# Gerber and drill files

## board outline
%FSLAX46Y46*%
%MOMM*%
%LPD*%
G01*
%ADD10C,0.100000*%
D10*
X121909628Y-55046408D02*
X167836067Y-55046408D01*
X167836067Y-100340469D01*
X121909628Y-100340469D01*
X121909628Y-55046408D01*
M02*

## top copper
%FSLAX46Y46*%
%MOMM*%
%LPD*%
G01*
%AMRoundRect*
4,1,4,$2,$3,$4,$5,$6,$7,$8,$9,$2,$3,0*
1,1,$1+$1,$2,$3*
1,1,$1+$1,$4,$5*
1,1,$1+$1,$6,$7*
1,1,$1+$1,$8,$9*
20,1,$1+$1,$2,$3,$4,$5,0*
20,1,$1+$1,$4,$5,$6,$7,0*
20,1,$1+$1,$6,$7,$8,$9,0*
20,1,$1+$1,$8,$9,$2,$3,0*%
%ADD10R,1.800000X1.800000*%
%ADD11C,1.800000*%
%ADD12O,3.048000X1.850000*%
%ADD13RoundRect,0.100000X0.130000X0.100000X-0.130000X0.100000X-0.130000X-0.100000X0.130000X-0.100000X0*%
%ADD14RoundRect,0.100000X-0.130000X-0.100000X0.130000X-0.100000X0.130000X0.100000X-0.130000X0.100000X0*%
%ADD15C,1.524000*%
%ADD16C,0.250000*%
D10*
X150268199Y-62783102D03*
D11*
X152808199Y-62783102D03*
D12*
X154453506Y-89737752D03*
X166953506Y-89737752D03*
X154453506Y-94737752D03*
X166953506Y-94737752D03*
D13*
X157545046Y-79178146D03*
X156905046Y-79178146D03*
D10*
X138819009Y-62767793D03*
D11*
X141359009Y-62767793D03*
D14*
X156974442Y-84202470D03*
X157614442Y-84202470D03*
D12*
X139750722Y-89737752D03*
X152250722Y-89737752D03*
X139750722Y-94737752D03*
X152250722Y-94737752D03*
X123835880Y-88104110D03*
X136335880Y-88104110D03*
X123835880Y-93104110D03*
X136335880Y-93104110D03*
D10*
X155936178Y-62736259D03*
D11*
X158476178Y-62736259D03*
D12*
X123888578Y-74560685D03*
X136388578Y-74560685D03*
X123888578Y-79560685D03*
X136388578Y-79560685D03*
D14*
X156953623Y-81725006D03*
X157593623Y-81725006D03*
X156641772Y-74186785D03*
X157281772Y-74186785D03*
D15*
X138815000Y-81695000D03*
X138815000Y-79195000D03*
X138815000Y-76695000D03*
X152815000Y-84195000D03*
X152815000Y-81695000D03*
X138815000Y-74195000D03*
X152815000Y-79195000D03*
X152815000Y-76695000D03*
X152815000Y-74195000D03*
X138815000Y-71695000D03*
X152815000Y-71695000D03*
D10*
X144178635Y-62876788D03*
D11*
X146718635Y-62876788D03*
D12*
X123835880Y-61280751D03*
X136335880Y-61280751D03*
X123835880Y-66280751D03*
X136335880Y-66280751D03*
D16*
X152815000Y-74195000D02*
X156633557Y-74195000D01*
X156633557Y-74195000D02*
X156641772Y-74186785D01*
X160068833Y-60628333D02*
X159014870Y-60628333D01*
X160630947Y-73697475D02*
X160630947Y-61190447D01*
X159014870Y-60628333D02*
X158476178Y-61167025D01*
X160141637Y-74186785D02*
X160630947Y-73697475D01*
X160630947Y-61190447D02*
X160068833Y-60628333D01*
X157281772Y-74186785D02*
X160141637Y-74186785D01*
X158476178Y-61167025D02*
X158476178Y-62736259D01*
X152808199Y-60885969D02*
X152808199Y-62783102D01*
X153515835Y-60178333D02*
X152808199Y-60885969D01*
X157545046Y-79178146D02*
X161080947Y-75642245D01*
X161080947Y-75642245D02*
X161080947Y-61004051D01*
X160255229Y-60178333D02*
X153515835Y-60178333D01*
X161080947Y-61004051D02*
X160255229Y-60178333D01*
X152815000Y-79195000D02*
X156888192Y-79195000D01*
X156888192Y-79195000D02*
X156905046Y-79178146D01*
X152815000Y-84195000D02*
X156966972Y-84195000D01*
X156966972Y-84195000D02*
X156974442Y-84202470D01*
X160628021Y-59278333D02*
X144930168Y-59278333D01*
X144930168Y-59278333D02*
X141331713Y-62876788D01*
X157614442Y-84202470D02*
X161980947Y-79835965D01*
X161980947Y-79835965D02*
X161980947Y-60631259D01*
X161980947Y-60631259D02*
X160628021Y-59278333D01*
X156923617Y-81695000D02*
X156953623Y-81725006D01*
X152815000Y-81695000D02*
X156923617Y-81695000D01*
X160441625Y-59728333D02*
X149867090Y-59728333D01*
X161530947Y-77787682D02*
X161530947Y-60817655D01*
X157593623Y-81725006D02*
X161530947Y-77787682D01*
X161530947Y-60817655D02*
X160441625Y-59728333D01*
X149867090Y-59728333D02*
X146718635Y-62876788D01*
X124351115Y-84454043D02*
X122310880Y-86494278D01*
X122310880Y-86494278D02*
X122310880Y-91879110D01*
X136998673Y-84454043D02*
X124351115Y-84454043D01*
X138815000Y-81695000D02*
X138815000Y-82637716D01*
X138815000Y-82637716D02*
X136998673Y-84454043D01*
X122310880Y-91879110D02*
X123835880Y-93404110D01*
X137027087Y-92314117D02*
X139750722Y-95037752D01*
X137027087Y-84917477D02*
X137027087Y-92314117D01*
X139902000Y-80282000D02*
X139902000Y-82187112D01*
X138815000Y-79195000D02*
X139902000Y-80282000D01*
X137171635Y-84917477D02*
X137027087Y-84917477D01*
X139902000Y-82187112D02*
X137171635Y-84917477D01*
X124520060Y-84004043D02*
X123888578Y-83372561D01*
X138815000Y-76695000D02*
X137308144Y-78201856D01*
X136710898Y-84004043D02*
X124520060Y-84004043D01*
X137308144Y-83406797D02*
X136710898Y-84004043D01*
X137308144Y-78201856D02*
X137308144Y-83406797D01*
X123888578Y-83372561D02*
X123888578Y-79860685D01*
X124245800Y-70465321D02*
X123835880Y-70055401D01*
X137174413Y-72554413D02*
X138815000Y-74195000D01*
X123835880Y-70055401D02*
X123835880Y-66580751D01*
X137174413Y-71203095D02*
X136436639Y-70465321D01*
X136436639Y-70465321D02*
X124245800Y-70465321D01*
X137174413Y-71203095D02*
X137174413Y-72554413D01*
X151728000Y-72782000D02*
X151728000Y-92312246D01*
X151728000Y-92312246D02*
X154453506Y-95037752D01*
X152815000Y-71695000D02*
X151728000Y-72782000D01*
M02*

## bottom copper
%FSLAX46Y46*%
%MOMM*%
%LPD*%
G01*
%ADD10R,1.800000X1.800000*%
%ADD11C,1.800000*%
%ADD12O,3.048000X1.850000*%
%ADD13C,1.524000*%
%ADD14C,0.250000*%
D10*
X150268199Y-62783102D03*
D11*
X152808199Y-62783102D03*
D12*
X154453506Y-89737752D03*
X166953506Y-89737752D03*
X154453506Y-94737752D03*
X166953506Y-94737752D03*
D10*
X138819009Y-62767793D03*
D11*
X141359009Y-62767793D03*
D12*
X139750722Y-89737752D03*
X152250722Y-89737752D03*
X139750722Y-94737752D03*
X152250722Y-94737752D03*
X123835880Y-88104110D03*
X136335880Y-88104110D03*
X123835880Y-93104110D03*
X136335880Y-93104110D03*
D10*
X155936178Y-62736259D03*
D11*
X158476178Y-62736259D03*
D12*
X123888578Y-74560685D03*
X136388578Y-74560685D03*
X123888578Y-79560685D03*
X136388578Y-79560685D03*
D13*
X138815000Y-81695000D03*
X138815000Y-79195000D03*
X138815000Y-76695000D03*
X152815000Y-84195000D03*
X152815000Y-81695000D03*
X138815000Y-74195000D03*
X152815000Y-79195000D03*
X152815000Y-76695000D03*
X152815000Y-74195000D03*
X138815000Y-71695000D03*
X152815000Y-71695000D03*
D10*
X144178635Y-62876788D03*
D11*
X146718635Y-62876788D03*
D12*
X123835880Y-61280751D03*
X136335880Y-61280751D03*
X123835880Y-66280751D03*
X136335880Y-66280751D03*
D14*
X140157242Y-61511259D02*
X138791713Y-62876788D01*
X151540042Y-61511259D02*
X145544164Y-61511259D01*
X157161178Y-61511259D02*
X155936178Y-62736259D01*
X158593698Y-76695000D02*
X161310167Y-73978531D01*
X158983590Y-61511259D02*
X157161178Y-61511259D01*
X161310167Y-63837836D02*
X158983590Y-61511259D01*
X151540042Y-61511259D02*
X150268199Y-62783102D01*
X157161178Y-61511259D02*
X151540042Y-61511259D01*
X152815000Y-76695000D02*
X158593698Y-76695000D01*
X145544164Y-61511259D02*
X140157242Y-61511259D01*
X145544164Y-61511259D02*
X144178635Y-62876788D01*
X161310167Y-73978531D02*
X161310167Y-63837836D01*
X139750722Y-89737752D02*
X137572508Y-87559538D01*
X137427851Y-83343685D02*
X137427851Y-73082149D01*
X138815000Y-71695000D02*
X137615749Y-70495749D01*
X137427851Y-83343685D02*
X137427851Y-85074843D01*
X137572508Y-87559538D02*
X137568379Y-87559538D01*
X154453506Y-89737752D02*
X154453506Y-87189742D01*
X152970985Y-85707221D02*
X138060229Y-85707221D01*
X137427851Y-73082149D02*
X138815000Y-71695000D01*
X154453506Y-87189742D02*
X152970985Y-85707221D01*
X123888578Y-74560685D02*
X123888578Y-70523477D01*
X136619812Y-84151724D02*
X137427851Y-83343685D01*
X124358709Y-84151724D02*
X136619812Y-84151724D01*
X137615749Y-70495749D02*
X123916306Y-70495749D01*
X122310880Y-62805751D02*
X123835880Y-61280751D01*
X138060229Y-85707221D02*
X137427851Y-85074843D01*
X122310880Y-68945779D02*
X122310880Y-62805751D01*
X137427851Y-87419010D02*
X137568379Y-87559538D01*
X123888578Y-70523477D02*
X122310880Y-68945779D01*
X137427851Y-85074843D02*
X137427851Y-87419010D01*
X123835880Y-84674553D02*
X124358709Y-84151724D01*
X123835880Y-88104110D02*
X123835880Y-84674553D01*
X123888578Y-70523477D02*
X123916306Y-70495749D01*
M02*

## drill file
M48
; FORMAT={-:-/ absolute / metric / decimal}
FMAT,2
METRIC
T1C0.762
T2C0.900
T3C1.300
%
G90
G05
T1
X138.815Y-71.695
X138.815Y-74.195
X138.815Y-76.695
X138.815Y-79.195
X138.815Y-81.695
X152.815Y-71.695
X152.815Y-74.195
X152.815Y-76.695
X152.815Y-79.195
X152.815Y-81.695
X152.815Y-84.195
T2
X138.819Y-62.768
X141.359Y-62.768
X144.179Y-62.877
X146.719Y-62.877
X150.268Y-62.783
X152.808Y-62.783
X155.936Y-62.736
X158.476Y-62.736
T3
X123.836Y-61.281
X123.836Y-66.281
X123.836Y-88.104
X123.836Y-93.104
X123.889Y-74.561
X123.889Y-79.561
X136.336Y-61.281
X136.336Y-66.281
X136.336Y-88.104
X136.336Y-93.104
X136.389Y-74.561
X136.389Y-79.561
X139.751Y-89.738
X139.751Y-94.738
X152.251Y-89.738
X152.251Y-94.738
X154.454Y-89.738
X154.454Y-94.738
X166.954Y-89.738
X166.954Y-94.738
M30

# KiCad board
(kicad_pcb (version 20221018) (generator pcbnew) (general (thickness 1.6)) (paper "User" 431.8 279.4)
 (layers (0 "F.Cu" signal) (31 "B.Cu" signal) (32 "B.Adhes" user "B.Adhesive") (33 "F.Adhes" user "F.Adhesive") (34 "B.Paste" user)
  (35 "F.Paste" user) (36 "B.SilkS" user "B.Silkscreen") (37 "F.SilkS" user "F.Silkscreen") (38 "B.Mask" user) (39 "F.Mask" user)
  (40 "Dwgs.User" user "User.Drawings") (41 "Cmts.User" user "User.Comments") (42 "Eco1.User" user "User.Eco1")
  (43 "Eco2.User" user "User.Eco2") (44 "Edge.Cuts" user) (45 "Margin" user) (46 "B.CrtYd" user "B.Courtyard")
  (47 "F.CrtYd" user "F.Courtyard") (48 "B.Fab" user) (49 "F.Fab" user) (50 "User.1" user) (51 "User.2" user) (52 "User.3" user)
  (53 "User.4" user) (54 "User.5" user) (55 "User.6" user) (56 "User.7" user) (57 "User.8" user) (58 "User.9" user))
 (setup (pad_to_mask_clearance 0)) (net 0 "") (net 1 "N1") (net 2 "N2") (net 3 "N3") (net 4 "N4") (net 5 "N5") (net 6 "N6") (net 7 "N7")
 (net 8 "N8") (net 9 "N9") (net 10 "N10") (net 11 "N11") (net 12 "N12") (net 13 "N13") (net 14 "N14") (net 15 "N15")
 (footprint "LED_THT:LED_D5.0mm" (layer "F.Cu") (at 150.268199 62.783102)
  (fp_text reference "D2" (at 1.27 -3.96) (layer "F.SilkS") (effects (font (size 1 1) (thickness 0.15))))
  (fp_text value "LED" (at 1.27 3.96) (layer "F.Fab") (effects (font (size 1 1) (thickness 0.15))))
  (pad "1" thru_hole rect (at 0 0) (size 1.8 1.8) (drill 0.9) (layers "*.Cu" "*.Mask") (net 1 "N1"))
  (pad "2" thru_hole circle (at 2.54 0) (size 1.8 1.8) (drill 0.9) (layers "*.Cu" "*.Mask") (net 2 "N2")))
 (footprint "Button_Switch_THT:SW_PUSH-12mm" (layer "F.Cu") (at 154.453506 89.737752)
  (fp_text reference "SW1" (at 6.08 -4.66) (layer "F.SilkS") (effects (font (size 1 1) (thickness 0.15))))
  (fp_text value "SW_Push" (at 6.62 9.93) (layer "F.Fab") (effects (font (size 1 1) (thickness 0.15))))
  (pad "1" thru_hole oval (at 0 0) (size 3.048 1.85) (drill 1.3) (layers "*.Cu" "*.Mask") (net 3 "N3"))
  (pad "1" thru_hole oval (at 12.5 0) (size 3.048 1.85) (drill 1.3) (layers "*.Cu" "*.Mask") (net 3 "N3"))
  (pad "2" thru_hole oval (at 0 5) (size 3.048 1.85) (drill 1.3) (layers "*.Cu" "*.Mask") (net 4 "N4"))
  (pad "2" thru_hole oval (at 12.5 5) (size 3.048 1.85) (drill 1.3) (layers "*.Cu" "*.Mask") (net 4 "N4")))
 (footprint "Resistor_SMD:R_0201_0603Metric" (layer "F.Cu") (at 157.225046 79.178146 180)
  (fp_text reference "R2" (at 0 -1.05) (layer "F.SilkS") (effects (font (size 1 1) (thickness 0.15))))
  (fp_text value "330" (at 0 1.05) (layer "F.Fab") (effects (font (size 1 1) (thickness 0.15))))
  (pad "" smd roundrect (at -0.345 0 180) (size 0.318 0.36) (layers "F.Paste") (roundrect_rratio 0.25))
  (pad "" smd roundrect (at 0.345 0 180) (size 0.318 0.36) (layers "F.Paste") (roundrect_rratio 0.25))
  (pad "1" smd roundrect (at -0.32 0 180) (size 0.46 0.4) (layers "F.Cu" "F.Mask") (roundrect_rratio 0.25) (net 2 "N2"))
  (pad "2" smd roundrect (at 0.32 0 180) (size 0.46 0.4) (layers "F.Cu" "F.Mask") (roundrect_rratio 0.25) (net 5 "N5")))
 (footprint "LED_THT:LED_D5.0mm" (layer "F.Cu") (at 138.819009 62.767793)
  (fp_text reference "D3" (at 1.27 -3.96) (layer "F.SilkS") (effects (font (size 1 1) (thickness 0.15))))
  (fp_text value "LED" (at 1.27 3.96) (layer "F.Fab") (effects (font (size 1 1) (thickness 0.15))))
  (pad "1" thru_hole rect (at 0 0) (size 1.8 1.8) (drill 0.9) (layers "*.Cu" "*.Mask") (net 1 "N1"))
  (pad "2" thru_hole circle (at 2.54 0) (size 1.8 1.8) (drill 0.9) (layers "*.Cu" "*.Mask") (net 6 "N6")))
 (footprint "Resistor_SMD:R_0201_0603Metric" (layer "F.Cu") (at 157.294442 84.20247)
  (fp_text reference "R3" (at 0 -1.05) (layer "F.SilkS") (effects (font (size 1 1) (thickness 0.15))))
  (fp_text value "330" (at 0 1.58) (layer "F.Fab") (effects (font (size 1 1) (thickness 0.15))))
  (pad "" smd roundrect (at -0.345 0) (size 0.318 0.36) (layers "F.Paste") (roundrect_rratio 0.25))
  (pad "" smd roundrect (at 0.345 0) (size 0.318 0.36) (layers "F.Paste") (roundrect_rratio 0.25))
  (pad "1" smd roundrect (at -0.32 0) (size 0.46 0.4) (layers "F.Cu" "F.Mask") (roundrect_rratio 0.25) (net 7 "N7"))
  (pad "2" smd roundrect (at 0.32 0) (size 0.46 0.4) (layers "F.Cu" "F.Mask") (roundrect_rratio 0.25) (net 6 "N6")))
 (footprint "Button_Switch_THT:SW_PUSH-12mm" (layer "F.Cu") (at 139.750722 89.737752)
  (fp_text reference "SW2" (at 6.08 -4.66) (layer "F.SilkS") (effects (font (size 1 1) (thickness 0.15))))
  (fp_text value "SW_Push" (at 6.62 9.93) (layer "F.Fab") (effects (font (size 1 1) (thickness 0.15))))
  (pad "1" thru_hole oval (at 0 0) (size 3.048 1.85) (drill 1.3) (layers "*.Cu" "*.Mask") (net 3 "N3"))
  (pad "1" thru_hole oval (at 12.5 0) (size 3.048 1.85) (drill 1.3) (layers "*.Cu" "*.Mask") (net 3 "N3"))
  (pad "2" thru_hole oval (at 0 5) (size 3.048 1.85) (drill 1.3) (layers "*.Cu" "*.Mask") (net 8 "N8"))
  (pad "2" thru_hole oval (at 12.5 5) (size 3.048 1.85) (drill 1.3) (layers "*.Cu" "*.Mask") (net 8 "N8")))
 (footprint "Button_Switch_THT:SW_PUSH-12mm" (layer "F.Cu") (at 123.83588 88.10411)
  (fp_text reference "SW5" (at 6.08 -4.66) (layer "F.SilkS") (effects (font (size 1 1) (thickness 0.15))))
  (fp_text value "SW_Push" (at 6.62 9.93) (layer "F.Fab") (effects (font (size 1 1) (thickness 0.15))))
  (pad "1" thru_hole oval (at 0 0) (size 3.048 1.85) (drill 1.3) (layers "*.Cu" "*.Mask") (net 3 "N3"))
  (pad "1" thru_hole oval (at 12.5 0) (size 3.048 1.85) (drill 1.3) (layers "*.Cu" "*.Mask") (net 3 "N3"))
  (pad "2" thru_hole oval (at 0 5) (size 3.048 1.85) (drill 1.3) (layers "*.Cu" "*.Mask") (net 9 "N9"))
  (pad "2" thru_hole oval (at 12.5 5) (size 3.048 1.85) (drill 1.3) (layers "*.Cu" "*.Mask") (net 9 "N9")))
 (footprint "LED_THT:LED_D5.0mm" (layer "F.Cu") (at 155.936178 62.736259)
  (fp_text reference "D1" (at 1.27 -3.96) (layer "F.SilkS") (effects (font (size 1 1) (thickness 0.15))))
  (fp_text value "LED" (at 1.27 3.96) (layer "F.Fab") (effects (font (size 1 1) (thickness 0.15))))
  (pad "1" thru_hole rect (at 0 0) (size 1.8 1.8) (drill 0.9) (layers "*.Cu" "*.Mask") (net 1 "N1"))
  (pad "2" thru_hole circle (at 2.54 0) (size 1.8 1.8) (drill 0.9) (layers "*.Cu" "*.Mask") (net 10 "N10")))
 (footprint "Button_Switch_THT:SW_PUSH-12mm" (layer "F.Cu") (at 123.888578 74.560685)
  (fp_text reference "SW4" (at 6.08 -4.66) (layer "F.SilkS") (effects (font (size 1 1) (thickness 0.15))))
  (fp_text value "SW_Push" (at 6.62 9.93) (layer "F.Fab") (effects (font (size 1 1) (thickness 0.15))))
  (pad "1" thru_hole oval (at 0 0) (size 3.048 1.85) (drill 1.3) (layers "*.Cu" "*.Mask") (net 3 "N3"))
  (pad "1" thru_hole oval (at 12.5 0) (size 3.048 1.85) (drill 1.3) (layers "*.Cu" "*.Mask") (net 3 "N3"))
  (pad "2" thru_hole oval (at 0 5) (size 3.048 1.85) (drill 1.3) (layers "*.Cu" "*.Mask") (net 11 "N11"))
  (pad "2" thru_hole oval (at 12.5 5) (size 3.048 1.85) (drill 1.3) (layers "*.Cu" "*.Mask") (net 11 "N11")))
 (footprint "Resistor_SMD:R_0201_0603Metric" (layer "F.Cu") (at 157.273623 81.725006)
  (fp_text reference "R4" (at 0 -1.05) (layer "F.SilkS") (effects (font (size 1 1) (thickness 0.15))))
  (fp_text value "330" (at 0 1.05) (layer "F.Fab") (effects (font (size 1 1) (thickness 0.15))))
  (pad "" smd roundrect (at -0.345 0) (size 0.318 0.36) (layers "F.Paste") (roundrect_rratio 0.25))
  (pad "" smd roundrect (at 0.345 0) (size 0.318 0.36) (layers "F.Paste") (roundrect_rratio 0.25))
  (pad "1" smd roundrect (at -0.32 0) (size 0.46 0.4) (layers "F.Cu" "F.Mask") (roundrect_rratio 0.25) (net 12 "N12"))
  (pad "2" smd roundrect (at 0.32 0) (size 0.46 0.4) (layers "F.Cu" "F.Mask") (roundrect_rratio 0.25) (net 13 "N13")))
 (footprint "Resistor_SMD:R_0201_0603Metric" (layer "F.Cu") (at 156.961772 74.186785)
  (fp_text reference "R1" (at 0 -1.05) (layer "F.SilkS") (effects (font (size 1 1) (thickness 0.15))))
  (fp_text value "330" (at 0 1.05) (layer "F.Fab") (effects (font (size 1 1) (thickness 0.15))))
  (pad "" smd roundrect (at -0.345 0) (size 0.318 0.36) (layers "F.Paste") (roundrect_rratio 0.25))
  (pad "" smd roundrect (at 0.345 0) (size 0.318 0.36) (layers "F.Paste") (roundrect_rratio 0.25))
  (pad "1" smd roundrect (at -0.32 0) (size 0.46 0.4) (layers "F.Cu" "F.Mask") (roundrect_rratio 0.25) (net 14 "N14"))
  (pad "2" smd roundrect (at 0.32 0) (size 0.46 0.4) (layers "F.Cu" "F.Mask") (roundrect_rratio 0.25) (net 10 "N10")))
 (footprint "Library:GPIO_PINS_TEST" (layer "F.Cu") (at 145.815 75.695)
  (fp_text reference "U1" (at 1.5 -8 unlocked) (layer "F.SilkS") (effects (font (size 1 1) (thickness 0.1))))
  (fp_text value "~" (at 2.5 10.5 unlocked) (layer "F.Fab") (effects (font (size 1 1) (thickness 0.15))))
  (pad "3" thru_hole circle (at -7 6) (size 1.524 1.524) (drill 0.762) (layers "*.Cu" "*.Mask") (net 9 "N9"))
  (pad "5" thru_hole circle (at -7 3.5) (size 1.524 1.524) (drill 0.762) (layers "*.Cu" "*.Mask") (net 8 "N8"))
  (pad "7" thru_hole circle (at -7 1) (size 1.524 1.524) (drill 0.762) (layers "*.Cu" "*.Mask") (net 11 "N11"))
  (pad "8" thru_hole circle (at 7 8.5) (size 1.524 1.524) (drill 0.762) (layers "*.Cu" "*.Mask") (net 7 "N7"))
  (pad "10" thru_hole circle (at 7 6) (size 1.524 1.524) (drill 0.762) (layers "*.Cu" "*.Mask") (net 12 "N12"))
  (pad "19" thru_hole circle (at -7 -1.5) (size 1.524 1.524) (drill 0.762) (layers "*.Cu" "*.Mask") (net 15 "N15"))
  (pad "32" thru_hole circle (at 7 3.5) (size 1.524 1.524) (drill 0.762) (layers "*.Cu" "*.Mask") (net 5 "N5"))
  (pad "34" thru_hole circle (at 7 1) (size 1.524 1.524) (drill 0.762) (layers "*.Cu" "*.Mask") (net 1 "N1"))
  (pad "36" thru_hole circle (at 7 -1.5) (size 1.524 1.524) (drill 0.762) (layers "*.Cu" "*.Mask") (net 14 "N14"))
  (pad "39" thru_hole circle (at -7 -4) (size 1.524 1.524) (drill 0.762) (layers "*.Cu" "*.Mask") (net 3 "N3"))
  (pad "40" thru_hole circle (at 7 -4) (size 1.524 1.524) (drill 0.762) (layers "*.Cu" "*.Mask") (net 4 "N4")))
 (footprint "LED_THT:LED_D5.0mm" (layer "F.Cu") (at 144.178635 62.876788)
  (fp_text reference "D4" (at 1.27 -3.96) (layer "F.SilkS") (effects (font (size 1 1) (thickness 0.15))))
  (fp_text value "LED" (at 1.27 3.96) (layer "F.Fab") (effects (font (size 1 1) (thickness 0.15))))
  (pad "1" thru_hole rect (at 0 0) (size 1.8 1.8) (drill 0.9) (layers "*.Cu" "*.Mask") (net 1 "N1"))
  (pad "2" thru_hole circle (at 2.54 0) (size 1.8 1.8) (drill 0.9) (layers "*.Cu" "*.Mask") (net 13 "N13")))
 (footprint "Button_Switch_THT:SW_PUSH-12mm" (layer "F.Cu") (at 123.83588 61.280751)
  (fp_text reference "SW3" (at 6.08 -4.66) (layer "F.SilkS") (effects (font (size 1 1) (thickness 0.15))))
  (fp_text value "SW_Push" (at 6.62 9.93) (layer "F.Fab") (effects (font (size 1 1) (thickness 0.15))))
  (pad "1" thru_hole oval (at 0 0) (size 3.048 1.85) (drill 1.3) (layers "*.Cu" "*.Mask") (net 3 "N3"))
  (pad "1" thru_hole oval (at 12.5 0) (size 3.048 1.85) (drill 1.3) (layers "*.Cu" "*.Mask") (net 3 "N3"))
  (pad "2" thru_hole oval (at 0 5) (size 3.048 1.85) (drill 1.3) (layers "*.Cu" "*.Mask") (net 15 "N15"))
  (pad "2" thru_hole oval (at 12.5 5) (size 3.048 1.85) (drill 1.3) (layers "*.Cu" "*.Mask") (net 15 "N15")))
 (gr_rect (start 121.909628 55.046408) (end 167.836067 100.340469) (stroke (width 0.1) (type default)) (fill none) (layer "Edge.Cuts"))
 (segment (start 152.815 74.195) (end 156.633557 74.195) (width 0.25) (layer "F.Cu") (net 14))
 (segment (start 156.633557 74.195) (end 156.641772 74.186785) (width 0.25) (layer "F.Cu") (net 14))
 (segment (start 160.068833 60.628333) (end 159.01487 60.628333) (width 0.25) (layer "F.Cu") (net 10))
 (segment (start 160.630947 73.697475) (end 160.630947 61.190447) (width 0.25) (layer "F.Cu") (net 10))
 (segment (start 159.01487 60.628333) (end 158.476178 61.167025) (width 0.25) (layer "F.Cu") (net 10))
 (segment (start 160.141637 74.186785) (end 160.630947 73.697475) (width 0.25) (layer "F.Cu") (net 10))
 (segment (start 160.630947 61.190447) (end 160.068833 60.628333) (width 0.25) (layer "F.Cu") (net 10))
 (segment (start 157.281772 74.186785) (end 160.141637 74.186785) (width 0.25) (layer "F.Cu") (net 10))
 (segment (start 158.476178 61.167025) (end 158.476178 62.736259) (width 0.25) (layer "F.Cu") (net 10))
 (segment (start 152.808199 60.885969) (end 152.808199 62.783102) (width 0.25) (layer "F.Cu") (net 2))
 (segment (start 153.515835 60.178333) (end 152.808199 60.885969) (width 0.25) (layer "F.Cu") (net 2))
 (segment (start 157.545046 79.178146) (end 161.080947 75.642245) (width 0.25) (layer "F.Cu") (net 2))
 (segment (start 161.080947 75.642245) (end 161.080947 61.004051) (width 0.25) (layer "F.Cu") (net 2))
 (segment (start 160.255229 60.178333) (end 153.515835 60.178333) (width 0.25) (layer "F.Cu") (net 2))
 (segment (start 161.080947 61.004051) (end 160.255229 60.178333) (width 0.25) (layer "F.Cu") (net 2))
 (segment (start 152.815 79.195) (end 156.888192 79.195) (width 0.25) (layer "F.Cu") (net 5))
 (segment (start 156.888192 79.195) (end 156.905046 79.178146) (width 0.25) (layer "F.Cu") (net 5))
 (segment (start 152.815 84.195) (end 156.966972 84.195) (width 0.25) (layer "F.Cu") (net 7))
 (segment (start 156.966972 84.195) (end 156.974442 84.20247) (width 0.25) (layer "F.Cu") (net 7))
 (segment (start 160.628021 59.278333) (end 144.930168 59.278333) (width 0.25) (layer "F.Cu") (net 6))
 (segment (start 144.930168 59.278333) (end 141.331713 62.876788) (width 0.25) (layer "F.Cu") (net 6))
 (segment (start 157.614442 84.20247) (end 161.980947 79.835965) (width 0.25) (layer "F.Cu") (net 6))
 (segment (start 161.980947 79.835965) (end 161.980947 60.631259) (width 0.25) (layer "F.Cu") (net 6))
 (segment (start 161.980947 60.631259) (end 160.628021 59.278333) (width 0.25) (layer "F.Cu") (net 6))
 (segment (start 156.923617 81.695) (end 156.953623 81.725006) (width 0.25) (layer "F.Cu") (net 12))
 (segment (start 152.815 81.695) (end 156.923617 81.695) (width 0.25) (layer "F.Cu") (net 12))
 (segment (start 160.441625 59.728333) (end 149.86709 59.728333) (width 0.25) (layer "F.Cu") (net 13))
 (segment (start 161.530947 77.787682) (end 161.530947 60.817655) (width 0.25) (layer "F.Cu") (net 13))
 (segment (start 157.593623 81.725006) (end 161.530947 77.787682) (width 0.25) (layer "F.Cu") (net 13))
 (segment (start 161.530947 60.817655) (end 160.441625 59.728333) (width 0.25) (layer "F.Cu") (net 13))
 (segment (start 149.86709 59.728333) (end 146.718635 62.876788) (width 0.25) (layer "F.Cu") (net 13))
 (segment (start 124.351115 84.454043) (end 122.31088 86.494278) (width 0.25) (layer "F.Cu") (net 9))
 (segment (start 122.31088 86.494278) (end 122.31088 91.87911) (width 0.25) (layer "F.Cu") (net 9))
 (segment (start 136.998673 84.454043) (end 124.351115 84.454043) (width 0.25) (layer "F.Cu") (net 9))
 (segment (start 138.815 81.695) (end 138.815 82.637716) (width 0.25) (layer "F.Cu") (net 9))
 (segment (start 138.815 82.637716) (end 136.998673 84.454043) (width 0.25) (layer "F.Cu") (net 9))
 (segment (start 122.31088 91.87911) (end 123.83588 93.40411) (width 0.25) (layer "F.Cu") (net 9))
 (segment (start 137.027087 92.314117) (end 139.750722 95.037752) (width 0.25) (layer "F.Cu") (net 8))
 (segment (start 137.027087 84.917477) (end 137.027087 92.314117) (width 0.25) (layer "F.Cu") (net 8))
 (segment (start 139.902 80.282) (end 139.902 82.187112) (width 0.25) (layer "F.Cu") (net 8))
 (segment (start 138.815 79.195) (end 139.902 80.282) (width 0.25) (layer "F.Cu") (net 8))
 (segment (start 137.171635 84.917477) (end 137.027087 84.917477) (width 0.25) (layer "F.Cu") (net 8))
 (segment (start 139.902 82.187112) (end 137.171635 84.917477) (width 0.25) (layer "F.Cu") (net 8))
 (segment (start 124.52006 84.004043) (end 123.888578 83.372561) (width 0.25) (layer "F.Cu") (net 11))
 (segment (start 138.815 76.695) (end 137.308144 78.201856) (width 0.25) (layer "F.Cu") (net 11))
 (segment (start 136.710898 84.004043) (end 124.52006 84.004043) (width 0.25) (layer "F.Cu") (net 11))
 (segment (start 137.308144 83.406797) (end 136.710898 84.004043) (width 0.25) (layer "F.Cu") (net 11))
 (segment (start 137.308144 78.201856) (end 137.308144 83.406797) (width 0.25) (layer "F.Cu") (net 11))
 (segment (start 123.888578 83.372561) (end 123.888578 79.860685) (width 0.25) (layer "F.Cu") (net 11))
 (segment (start 124.2458 70.465321) (end 123.83588 70.055401) (width 0.25) (layer "F.Cu") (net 15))
 (segment (start 137.174413 72.554413) (end 138.815 74.195) (width 0.25) (layer "F.Cu") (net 15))
 (segment (start 123.83588 70.055401) (end 123.83588 66.580751) (width 0.25) (layer "F.Cu") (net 15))
 (segment (start 137.174413 71.203095) (end 136.436639 70.465321) (width 0.25) (layer "F.Cu") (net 15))
 (segment (start 136.436639 70.465321) (end 124.2458 70.465321) (width 0.25) (layer "F.Cu") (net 15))
 (segment (start 137.174413 71.203095) (end 137.174413 72.554413) (width 0.25) (layer "F.Cu") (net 15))
 (segment (start 140.157242 61.511259) (end 138.791713 62.876788) (width 0.25) (layer "B.Cu") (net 1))
 (segment (start 151.540042 61.511259) (end 145.544164 61.511259) (width 0.25) (layer "B.Cu") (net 1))
 (segment (start 157.161178 61.511259) (end 155.936178 62.736259) (width 0.25) (layer "B.Cu") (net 1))
 (segment (start 158.593698 76.695) (end 161.310167 73.978531) (width 0.25) (layer "B.Cu") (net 1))
 (segment (start 158.98359 61.511259) (end 157.161178 61.511259) (width 0.25) (layer "B.Cu") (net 1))
 (segment (start 161.310167 63.837836) (end 158.98359 61.511259) (width 0.25) (layer "B.Cu") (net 1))
 (segment (start 151.540042 61.511259) (end 150.268199 62.783102) (width 0.25) (layer "B.Cu") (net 1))
 (segment (start 157.161178 61.511259) (end 151.540042 61.511259) (width 0.25) (layer "B.Cu") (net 1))
 (segment (start 152.815 76.695) (end 158.593698 76.695) (width 0.25) (layer "B.Cu") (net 1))
 (segment (start 145.544164 61.511259) (end 140.157242 61.511259) (width 0.25) (layer "B.Cu") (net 1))
 (segment (start 145.544164 61.511259) (end 144.178635 62.876788) (width 0.25) (layer "B.Cu") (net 1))
 (segment (start 161.310167 73.978531) (end 161.310167 63.837836) (width 0.25) (layer "B.Cu") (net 1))
 (segment (start 139.750722 89.737752) (end 137.572508 87.559538) (width 0.25) (layer "B.Cu") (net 3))
 (segment (start 137.427851 83.343685) (end 137.427851 73.082149) (width 0.25) (layer "B.Cu") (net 3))
 (segment (start 138.815 71.695) (end 137.615749 70.495749) (width 0.25) (layer "B.Cu") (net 3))
 (segment (start 137.427851 83.343685) (end 137.427851 85.074843) (width 0.25) (layer "B.Cu") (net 3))
 (segment (start 137.572508 87.559538) (end 137.568379 87.559538) (width 0.25) (layer "B.Cu") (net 3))
 (segment (start 154.453506 89.737752) (end 154.453506 87.189742) (width 0.25) (layer "B.Cu") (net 3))
 (segment (start 152.970985 85.707221) (end 138.060229 85.707221) (width 0.25) (layer "B.Cu") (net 3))
 (segment (start 137.427851 73.082149) (end 138.815 71.695) (width 0.25) (layer "B.Cu") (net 3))
 (segment (start 154.453506 87.189742) (end 152.970985 85.707221) (width 0.25) (layer "B.Cu") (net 3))
 (segment (start 123.888578 74.560685) (end 123.888578 70.523477) (width 0.25) (layer "B.Cu") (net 3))
 (segment (start 136.619812 84.151724) (end 137.427851 83.343685) (width 0.25) (layer "B.Cu") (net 3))
 (segment (start 124.358709 84.151724) (end 136.619812 84.151724) (width 0.25) (layer "B.Cu") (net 3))
 (segment (start 137.615749 70.495749) (end 123.916306 70.495749) (width 0.25) (layer "B.Cu") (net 3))
 (segment (start 122.31088 62.805751) (end 123.83588 61.280751) (width 0.25) (layer "B.Cu") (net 3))
 (segment (start 138.060229 85.707221) (end 137.427851 85.074843) (width 0.25) (layer "B.Cu") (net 3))
 (segment (start 122.31088 68.945779) (end 122.31088 62.805751) (width 0.25) (layer "B.Cu") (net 3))
 (segment (start 137.427851 87.41901) (end 137.568379 87.559538) (width 0.25) (layer "B.Cu") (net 3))
 (segment (start 123.888578 70.523477) (end 122.31088 68.945779) (width 0.25) (layer "B.Cu") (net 3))
 (segment (start 137.427851 85.074843) (end 137.427851 87.41901) (width 0.25) (layer "B.Cu") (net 3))
 (segment (start 123.83588 84.674553) (end 124.358709 84.151724) (width 0.25) (layer "B.Cu") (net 3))
 (segment (start 123.83588 88.10411) (end 123.83588 84.674553) (width 0.25) (layer "B.Cu") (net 3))
 (segment (start 123.888578 70.523477) (end 123.916306 70.495749) (width 0.25) (layer "B.Cu") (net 3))
 (segment (start 151.728 72.782) (end 151.728 92.312246) (width 0.25) (layer "F.Cu") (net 4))
 (segment (start 151.728 92.312246) (end 154.453506 95.037752) (width 0.25) (layer "F.Cu") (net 4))
 (segment (start 152.815 71.695) (end 151.728 72.782) (width 0.25) (layer "F.Cu") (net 4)))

